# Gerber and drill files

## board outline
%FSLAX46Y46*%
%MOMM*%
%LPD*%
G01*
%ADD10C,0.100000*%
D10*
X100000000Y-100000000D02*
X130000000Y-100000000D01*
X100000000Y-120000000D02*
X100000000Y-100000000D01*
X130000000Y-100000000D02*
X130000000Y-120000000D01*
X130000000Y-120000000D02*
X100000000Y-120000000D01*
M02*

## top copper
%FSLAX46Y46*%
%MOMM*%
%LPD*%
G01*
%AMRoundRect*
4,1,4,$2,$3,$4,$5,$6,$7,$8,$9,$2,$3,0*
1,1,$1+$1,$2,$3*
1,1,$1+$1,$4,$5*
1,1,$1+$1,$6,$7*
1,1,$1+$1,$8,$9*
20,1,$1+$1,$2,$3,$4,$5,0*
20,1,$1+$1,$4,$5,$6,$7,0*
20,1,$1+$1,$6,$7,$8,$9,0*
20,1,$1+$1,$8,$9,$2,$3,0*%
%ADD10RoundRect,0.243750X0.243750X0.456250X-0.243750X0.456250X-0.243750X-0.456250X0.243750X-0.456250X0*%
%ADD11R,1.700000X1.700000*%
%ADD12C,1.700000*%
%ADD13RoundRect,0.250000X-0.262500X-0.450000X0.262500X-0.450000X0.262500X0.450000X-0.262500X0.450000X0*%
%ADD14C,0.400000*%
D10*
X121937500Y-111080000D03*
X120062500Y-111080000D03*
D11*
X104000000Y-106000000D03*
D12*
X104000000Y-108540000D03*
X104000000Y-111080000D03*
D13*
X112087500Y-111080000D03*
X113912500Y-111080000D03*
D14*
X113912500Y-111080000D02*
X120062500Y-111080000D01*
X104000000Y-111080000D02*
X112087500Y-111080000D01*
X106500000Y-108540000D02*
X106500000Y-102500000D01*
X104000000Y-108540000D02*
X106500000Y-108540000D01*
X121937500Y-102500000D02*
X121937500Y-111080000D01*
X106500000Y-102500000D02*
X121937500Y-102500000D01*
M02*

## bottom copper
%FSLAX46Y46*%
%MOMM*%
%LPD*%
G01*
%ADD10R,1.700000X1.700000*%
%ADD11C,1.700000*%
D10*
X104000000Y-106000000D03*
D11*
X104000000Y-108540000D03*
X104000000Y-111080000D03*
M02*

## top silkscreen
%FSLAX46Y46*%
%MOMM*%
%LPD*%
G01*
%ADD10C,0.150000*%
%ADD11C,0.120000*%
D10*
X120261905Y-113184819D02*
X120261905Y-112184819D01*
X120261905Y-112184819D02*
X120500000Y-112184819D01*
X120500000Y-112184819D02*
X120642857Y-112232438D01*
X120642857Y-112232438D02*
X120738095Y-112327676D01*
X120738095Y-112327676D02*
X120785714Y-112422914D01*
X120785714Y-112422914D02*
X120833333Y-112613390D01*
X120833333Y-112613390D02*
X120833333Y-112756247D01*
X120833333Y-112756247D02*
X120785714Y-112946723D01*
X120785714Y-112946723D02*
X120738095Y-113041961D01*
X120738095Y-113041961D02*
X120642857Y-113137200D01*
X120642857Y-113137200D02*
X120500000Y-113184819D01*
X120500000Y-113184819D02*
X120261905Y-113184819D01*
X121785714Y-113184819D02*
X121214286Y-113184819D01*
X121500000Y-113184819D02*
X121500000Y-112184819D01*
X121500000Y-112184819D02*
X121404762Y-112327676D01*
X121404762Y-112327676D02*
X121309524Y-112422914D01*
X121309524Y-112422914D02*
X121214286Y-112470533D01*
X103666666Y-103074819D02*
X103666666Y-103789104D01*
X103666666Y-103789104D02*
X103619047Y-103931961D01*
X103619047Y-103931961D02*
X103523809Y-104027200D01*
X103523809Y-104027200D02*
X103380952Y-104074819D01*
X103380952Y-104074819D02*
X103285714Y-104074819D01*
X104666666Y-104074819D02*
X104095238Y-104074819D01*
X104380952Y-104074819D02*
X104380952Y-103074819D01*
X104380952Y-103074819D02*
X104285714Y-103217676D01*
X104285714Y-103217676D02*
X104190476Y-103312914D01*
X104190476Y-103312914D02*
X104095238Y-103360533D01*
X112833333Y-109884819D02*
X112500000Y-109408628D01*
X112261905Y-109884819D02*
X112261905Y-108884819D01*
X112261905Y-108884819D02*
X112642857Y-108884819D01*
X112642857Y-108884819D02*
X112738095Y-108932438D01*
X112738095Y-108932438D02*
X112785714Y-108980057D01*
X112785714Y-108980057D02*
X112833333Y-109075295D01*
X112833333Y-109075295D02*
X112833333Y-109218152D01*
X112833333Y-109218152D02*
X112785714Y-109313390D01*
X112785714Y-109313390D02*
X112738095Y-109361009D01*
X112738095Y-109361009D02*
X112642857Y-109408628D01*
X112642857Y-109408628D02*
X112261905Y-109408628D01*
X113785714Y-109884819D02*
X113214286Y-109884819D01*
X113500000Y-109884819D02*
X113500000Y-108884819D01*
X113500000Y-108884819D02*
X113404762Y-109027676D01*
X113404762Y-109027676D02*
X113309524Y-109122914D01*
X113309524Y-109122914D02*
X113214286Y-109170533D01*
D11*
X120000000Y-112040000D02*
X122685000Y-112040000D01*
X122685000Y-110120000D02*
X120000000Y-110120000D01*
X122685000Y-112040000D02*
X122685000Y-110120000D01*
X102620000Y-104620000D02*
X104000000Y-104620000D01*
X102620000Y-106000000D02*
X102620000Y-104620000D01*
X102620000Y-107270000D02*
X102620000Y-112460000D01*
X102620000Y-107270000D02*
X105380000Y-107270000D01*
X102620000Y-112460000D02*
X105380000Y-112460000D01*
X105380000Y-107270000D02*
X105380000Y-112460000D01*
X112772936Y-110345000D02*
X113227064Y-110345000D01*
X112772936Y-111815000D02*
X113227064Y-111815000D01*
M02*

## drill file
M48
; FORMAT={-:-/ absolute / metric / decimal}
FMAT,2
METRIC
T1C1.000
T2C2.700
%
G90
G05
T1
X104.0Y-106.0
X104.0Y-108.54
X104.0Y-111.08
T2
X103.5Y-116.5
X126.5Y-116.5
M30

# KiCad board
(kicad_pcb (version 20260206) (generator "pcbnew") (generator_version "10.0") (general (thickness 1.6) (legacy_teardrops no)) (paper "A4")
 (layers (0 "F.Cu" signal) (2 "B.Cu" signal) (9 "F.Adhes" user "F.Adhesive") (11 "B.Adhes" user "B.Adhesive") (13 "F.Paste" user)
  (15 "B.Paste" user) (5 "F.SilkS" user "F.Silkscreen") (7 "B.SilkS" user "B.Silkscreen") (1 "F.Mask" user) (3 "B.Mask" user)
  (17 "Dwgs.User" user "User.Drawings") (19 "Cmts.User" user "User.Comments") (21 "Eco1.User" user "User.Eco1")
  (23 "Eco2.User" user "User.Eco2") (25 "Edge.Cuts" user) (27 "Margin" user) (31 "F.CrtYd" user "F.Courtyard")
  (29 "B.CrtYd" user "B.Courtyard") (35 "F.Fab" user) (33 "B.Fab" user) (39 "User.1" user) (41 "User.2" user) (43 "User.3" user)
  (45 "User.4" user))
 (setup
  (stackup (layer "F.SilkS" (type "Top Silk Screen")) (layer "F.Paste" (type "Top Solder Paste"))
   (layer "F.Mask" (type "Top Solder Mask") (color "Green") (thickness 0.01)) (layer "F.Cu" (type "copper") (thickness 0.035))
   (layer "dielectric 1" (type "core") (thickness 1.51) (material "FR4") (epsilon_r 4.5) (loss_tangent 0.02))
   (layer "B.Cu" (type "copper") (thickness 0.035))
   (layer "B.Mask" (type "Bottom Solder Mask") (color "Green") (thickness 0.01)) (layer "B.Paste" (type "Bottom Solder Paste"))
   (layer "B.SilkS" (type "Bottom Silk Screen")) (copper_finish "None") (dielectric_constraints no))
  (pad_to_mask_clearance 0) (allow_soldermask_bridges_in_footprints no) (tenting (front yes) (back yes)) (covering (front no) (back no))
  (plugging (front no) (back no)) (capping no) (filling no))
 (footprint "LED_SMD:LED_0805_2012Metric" (layer "F.Cu") (at 121 111.08 180)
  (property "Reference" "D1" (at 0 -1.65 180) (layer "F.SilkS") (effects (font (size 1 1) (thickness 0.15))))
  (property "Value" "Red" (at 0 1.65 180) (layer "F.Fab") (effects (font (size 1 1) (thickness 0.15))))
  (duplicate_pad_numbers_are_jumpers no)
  (fp_line (start 1 -0.96) (end -1.685 -0.96) (stroke (width 0.12) (type solid)) (layer "F.SilkS"))
  (fp_line (start -1.685 0.96) (end 1 0.96) (stroke (width 0.12) (type solid)) (layer "F.SilkS"))
  (fp_line (start -1.685 -0.96) (end -1.685 0.96) (stroke (width 0.12) (type solid)) (layer "F.SilkS"))
  (pad "1" smd roundrect (at -0.9375 0 180) (size 0.975 1.4) (layers "F.Cu" "F.Mask" "F.Paste") (roundrect_rratio 0.25) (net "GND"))
  (pad "2" smd roundrect (at 0.9375 0 180) (size 0.975 1.4) (layers "F.Cu" "F.Mask" "F.Paste") (roundrect_rratio 0.25) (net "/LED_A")))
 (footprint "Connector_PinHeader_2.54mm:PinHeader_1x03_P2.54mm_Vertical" (layer "F.Cu") (at 104 106)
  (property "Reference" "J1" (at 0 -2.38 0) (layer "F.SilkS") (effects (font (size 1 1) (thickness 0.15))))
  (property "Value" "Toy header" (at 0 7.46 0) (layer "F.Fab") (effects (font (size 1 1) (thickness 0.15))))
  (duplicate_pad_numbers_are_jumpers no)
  (fp_line (start -1.38 -1.38) (end 0 -1.38) (stroke (width 0.12) (type solid)) (layer "F.SilkS"))
  (fp_line (start -1.38 0) (end -1.38 -1.38) (stroke (width 0.12) (type solid)) (layer "F.SilkS"))
  (fp_line (start -1.38 1.27) (end -1.38 6.46) (stroke (width 0.12) (type solid)) (layer "F.SilkS"))
  (fp_line (start -1.38 1.27) (end 1.38 1.27) (stroke (width 0.12) (type solid)) (layer "F.SilkS"))
  (fp_line (start -1.38 6.46) (end 1.38 6.46) (stroke (width 0.12) (type solid)) (layer "F.SilkS"))
  (fp_line (start 1.38 1.27) (end 1.38 6.46) (stroke (width 0.12) (type solid)) (layer "F.SilkS"))
  (pad "1" thru_hole rect (at 0 0) (size 1.7 1.7) (drill 1) (layers "*.Cu" "*.Mask") (remove_unused_layers no) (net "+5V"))
  (pad "2" thru_hole circle (at 0 2.54) (size 1.7 1.7) (drill 1) (layers "*.Cu" "*.Mask") (remove_unused_layers no) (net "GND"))
  (pad "3" thru_hole circle (at 0 5.08) (size 1.7 1.7) (drill 1) (layers "*.Cu" "*.Mask") (remove_unused_layers no) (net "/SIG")))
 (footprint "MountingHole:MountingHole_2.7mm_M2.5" (layer "F.Cu") (at 126.5 116.5)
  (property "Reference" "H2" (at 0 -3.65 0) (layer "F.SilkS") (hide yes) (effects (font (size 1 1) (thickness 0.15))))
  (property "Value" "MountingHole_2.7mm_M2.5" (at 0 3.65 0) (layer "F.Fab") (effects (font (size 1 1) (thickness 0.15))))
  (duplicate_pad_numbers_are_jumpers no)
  (pad "" np_thru_hole circle (at 0 0) (size 2.7 2.7) (drill 2.7) (layers "*.Cu" "*.Mask")))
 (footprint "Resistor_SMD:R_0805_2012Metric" (layer "F.Cu") (at 113 111.08)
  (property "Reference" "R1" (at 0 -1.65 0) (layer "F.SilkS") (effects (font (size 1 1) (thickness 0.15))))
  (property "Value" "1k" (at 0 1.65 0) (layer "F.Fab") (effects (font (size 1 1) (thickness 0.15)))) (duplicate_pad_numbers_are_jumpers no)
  (fp_line (start -0.227064 -0.735) (end 0.227064 -0.735) (stroke (width 0.12) (type solid)) (layer "F.SilkS"))
  (fp_line (start -0.227064 0.735) (end 0.227064 0.735) (stroke (width 0.12) (type solid)) (layer "F.SilkS"))
  (pad "1" smd roundrect (at -0.9125 0) (size 1.025 1.4) (layers "F.Cu" "F.Mask" "F.Paste") (roundrect_rratio 0.243902) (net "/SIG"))
  (pad "2" smd roundrect (at 0.9125 0) (size 1.025 1.4) (layers "F.Cu" "F.Mask" "F.Paste") (roundrect_rratio 0.243902) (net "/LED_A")))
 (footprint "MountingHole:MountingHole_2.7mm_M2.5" (layer "F.Cu") (at 103.5 116.5)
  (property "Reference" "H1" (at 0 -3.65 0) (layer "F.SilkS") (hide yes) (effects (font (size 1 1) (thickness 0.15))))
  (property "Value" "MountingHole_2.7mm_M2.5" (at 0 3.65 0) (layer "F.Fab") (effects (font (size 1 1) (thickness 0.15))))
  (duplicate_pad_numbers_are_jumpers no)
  (pad "" np_thru_hole circle (at 0 0) (size 2.7 2.7) (drill 2.7) (layers "*.Cu" "*.Mask")))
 (gr_line (start 100 100) (end 130 100) (stroke (width 0.1) (type default)) (layer "Edge.Cuts"))
 (gr_line (start 100 120) (end 100 100) (stroke (width 0.1) (type default)) (layer "Edge.Cuts"))
 (gr_line (start 130 100) (end 130 120) (stroke (width 0.1) (type default)) (layer "Edge.Cuts"))
 (gr_line (start 130 120) (end 100 120) (stroke (width 0.1) (type default)) (layer "Edge.Cuts"))
 (segment (start 113.9125 111.08) (end 120.0625 111.08) (width 0.4) (layer "F.Cu") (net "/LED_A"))
 (segment (start 104 111.08) (end 112.0875 111.08) (width 0.4) (layer "F.Cu") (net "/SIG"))
 (segment (start 106.5 108.54) (end 106.5 102.5) (width 0.4) (layer "F.Cu") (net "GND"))
 (segment (start 104 108.54) (end 106.5 108.54) (width 0.4) (layer "F.Cu") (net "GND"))
 (segment (start 121.9375 102.5) (end 121.9375 111.08) (width 0.4) (layer "F.Cu") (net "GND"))
 (segment (start 106.5 102.5) (end 121.9375 102.5) (width 0.4) (layer "F.Cu") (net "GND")))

